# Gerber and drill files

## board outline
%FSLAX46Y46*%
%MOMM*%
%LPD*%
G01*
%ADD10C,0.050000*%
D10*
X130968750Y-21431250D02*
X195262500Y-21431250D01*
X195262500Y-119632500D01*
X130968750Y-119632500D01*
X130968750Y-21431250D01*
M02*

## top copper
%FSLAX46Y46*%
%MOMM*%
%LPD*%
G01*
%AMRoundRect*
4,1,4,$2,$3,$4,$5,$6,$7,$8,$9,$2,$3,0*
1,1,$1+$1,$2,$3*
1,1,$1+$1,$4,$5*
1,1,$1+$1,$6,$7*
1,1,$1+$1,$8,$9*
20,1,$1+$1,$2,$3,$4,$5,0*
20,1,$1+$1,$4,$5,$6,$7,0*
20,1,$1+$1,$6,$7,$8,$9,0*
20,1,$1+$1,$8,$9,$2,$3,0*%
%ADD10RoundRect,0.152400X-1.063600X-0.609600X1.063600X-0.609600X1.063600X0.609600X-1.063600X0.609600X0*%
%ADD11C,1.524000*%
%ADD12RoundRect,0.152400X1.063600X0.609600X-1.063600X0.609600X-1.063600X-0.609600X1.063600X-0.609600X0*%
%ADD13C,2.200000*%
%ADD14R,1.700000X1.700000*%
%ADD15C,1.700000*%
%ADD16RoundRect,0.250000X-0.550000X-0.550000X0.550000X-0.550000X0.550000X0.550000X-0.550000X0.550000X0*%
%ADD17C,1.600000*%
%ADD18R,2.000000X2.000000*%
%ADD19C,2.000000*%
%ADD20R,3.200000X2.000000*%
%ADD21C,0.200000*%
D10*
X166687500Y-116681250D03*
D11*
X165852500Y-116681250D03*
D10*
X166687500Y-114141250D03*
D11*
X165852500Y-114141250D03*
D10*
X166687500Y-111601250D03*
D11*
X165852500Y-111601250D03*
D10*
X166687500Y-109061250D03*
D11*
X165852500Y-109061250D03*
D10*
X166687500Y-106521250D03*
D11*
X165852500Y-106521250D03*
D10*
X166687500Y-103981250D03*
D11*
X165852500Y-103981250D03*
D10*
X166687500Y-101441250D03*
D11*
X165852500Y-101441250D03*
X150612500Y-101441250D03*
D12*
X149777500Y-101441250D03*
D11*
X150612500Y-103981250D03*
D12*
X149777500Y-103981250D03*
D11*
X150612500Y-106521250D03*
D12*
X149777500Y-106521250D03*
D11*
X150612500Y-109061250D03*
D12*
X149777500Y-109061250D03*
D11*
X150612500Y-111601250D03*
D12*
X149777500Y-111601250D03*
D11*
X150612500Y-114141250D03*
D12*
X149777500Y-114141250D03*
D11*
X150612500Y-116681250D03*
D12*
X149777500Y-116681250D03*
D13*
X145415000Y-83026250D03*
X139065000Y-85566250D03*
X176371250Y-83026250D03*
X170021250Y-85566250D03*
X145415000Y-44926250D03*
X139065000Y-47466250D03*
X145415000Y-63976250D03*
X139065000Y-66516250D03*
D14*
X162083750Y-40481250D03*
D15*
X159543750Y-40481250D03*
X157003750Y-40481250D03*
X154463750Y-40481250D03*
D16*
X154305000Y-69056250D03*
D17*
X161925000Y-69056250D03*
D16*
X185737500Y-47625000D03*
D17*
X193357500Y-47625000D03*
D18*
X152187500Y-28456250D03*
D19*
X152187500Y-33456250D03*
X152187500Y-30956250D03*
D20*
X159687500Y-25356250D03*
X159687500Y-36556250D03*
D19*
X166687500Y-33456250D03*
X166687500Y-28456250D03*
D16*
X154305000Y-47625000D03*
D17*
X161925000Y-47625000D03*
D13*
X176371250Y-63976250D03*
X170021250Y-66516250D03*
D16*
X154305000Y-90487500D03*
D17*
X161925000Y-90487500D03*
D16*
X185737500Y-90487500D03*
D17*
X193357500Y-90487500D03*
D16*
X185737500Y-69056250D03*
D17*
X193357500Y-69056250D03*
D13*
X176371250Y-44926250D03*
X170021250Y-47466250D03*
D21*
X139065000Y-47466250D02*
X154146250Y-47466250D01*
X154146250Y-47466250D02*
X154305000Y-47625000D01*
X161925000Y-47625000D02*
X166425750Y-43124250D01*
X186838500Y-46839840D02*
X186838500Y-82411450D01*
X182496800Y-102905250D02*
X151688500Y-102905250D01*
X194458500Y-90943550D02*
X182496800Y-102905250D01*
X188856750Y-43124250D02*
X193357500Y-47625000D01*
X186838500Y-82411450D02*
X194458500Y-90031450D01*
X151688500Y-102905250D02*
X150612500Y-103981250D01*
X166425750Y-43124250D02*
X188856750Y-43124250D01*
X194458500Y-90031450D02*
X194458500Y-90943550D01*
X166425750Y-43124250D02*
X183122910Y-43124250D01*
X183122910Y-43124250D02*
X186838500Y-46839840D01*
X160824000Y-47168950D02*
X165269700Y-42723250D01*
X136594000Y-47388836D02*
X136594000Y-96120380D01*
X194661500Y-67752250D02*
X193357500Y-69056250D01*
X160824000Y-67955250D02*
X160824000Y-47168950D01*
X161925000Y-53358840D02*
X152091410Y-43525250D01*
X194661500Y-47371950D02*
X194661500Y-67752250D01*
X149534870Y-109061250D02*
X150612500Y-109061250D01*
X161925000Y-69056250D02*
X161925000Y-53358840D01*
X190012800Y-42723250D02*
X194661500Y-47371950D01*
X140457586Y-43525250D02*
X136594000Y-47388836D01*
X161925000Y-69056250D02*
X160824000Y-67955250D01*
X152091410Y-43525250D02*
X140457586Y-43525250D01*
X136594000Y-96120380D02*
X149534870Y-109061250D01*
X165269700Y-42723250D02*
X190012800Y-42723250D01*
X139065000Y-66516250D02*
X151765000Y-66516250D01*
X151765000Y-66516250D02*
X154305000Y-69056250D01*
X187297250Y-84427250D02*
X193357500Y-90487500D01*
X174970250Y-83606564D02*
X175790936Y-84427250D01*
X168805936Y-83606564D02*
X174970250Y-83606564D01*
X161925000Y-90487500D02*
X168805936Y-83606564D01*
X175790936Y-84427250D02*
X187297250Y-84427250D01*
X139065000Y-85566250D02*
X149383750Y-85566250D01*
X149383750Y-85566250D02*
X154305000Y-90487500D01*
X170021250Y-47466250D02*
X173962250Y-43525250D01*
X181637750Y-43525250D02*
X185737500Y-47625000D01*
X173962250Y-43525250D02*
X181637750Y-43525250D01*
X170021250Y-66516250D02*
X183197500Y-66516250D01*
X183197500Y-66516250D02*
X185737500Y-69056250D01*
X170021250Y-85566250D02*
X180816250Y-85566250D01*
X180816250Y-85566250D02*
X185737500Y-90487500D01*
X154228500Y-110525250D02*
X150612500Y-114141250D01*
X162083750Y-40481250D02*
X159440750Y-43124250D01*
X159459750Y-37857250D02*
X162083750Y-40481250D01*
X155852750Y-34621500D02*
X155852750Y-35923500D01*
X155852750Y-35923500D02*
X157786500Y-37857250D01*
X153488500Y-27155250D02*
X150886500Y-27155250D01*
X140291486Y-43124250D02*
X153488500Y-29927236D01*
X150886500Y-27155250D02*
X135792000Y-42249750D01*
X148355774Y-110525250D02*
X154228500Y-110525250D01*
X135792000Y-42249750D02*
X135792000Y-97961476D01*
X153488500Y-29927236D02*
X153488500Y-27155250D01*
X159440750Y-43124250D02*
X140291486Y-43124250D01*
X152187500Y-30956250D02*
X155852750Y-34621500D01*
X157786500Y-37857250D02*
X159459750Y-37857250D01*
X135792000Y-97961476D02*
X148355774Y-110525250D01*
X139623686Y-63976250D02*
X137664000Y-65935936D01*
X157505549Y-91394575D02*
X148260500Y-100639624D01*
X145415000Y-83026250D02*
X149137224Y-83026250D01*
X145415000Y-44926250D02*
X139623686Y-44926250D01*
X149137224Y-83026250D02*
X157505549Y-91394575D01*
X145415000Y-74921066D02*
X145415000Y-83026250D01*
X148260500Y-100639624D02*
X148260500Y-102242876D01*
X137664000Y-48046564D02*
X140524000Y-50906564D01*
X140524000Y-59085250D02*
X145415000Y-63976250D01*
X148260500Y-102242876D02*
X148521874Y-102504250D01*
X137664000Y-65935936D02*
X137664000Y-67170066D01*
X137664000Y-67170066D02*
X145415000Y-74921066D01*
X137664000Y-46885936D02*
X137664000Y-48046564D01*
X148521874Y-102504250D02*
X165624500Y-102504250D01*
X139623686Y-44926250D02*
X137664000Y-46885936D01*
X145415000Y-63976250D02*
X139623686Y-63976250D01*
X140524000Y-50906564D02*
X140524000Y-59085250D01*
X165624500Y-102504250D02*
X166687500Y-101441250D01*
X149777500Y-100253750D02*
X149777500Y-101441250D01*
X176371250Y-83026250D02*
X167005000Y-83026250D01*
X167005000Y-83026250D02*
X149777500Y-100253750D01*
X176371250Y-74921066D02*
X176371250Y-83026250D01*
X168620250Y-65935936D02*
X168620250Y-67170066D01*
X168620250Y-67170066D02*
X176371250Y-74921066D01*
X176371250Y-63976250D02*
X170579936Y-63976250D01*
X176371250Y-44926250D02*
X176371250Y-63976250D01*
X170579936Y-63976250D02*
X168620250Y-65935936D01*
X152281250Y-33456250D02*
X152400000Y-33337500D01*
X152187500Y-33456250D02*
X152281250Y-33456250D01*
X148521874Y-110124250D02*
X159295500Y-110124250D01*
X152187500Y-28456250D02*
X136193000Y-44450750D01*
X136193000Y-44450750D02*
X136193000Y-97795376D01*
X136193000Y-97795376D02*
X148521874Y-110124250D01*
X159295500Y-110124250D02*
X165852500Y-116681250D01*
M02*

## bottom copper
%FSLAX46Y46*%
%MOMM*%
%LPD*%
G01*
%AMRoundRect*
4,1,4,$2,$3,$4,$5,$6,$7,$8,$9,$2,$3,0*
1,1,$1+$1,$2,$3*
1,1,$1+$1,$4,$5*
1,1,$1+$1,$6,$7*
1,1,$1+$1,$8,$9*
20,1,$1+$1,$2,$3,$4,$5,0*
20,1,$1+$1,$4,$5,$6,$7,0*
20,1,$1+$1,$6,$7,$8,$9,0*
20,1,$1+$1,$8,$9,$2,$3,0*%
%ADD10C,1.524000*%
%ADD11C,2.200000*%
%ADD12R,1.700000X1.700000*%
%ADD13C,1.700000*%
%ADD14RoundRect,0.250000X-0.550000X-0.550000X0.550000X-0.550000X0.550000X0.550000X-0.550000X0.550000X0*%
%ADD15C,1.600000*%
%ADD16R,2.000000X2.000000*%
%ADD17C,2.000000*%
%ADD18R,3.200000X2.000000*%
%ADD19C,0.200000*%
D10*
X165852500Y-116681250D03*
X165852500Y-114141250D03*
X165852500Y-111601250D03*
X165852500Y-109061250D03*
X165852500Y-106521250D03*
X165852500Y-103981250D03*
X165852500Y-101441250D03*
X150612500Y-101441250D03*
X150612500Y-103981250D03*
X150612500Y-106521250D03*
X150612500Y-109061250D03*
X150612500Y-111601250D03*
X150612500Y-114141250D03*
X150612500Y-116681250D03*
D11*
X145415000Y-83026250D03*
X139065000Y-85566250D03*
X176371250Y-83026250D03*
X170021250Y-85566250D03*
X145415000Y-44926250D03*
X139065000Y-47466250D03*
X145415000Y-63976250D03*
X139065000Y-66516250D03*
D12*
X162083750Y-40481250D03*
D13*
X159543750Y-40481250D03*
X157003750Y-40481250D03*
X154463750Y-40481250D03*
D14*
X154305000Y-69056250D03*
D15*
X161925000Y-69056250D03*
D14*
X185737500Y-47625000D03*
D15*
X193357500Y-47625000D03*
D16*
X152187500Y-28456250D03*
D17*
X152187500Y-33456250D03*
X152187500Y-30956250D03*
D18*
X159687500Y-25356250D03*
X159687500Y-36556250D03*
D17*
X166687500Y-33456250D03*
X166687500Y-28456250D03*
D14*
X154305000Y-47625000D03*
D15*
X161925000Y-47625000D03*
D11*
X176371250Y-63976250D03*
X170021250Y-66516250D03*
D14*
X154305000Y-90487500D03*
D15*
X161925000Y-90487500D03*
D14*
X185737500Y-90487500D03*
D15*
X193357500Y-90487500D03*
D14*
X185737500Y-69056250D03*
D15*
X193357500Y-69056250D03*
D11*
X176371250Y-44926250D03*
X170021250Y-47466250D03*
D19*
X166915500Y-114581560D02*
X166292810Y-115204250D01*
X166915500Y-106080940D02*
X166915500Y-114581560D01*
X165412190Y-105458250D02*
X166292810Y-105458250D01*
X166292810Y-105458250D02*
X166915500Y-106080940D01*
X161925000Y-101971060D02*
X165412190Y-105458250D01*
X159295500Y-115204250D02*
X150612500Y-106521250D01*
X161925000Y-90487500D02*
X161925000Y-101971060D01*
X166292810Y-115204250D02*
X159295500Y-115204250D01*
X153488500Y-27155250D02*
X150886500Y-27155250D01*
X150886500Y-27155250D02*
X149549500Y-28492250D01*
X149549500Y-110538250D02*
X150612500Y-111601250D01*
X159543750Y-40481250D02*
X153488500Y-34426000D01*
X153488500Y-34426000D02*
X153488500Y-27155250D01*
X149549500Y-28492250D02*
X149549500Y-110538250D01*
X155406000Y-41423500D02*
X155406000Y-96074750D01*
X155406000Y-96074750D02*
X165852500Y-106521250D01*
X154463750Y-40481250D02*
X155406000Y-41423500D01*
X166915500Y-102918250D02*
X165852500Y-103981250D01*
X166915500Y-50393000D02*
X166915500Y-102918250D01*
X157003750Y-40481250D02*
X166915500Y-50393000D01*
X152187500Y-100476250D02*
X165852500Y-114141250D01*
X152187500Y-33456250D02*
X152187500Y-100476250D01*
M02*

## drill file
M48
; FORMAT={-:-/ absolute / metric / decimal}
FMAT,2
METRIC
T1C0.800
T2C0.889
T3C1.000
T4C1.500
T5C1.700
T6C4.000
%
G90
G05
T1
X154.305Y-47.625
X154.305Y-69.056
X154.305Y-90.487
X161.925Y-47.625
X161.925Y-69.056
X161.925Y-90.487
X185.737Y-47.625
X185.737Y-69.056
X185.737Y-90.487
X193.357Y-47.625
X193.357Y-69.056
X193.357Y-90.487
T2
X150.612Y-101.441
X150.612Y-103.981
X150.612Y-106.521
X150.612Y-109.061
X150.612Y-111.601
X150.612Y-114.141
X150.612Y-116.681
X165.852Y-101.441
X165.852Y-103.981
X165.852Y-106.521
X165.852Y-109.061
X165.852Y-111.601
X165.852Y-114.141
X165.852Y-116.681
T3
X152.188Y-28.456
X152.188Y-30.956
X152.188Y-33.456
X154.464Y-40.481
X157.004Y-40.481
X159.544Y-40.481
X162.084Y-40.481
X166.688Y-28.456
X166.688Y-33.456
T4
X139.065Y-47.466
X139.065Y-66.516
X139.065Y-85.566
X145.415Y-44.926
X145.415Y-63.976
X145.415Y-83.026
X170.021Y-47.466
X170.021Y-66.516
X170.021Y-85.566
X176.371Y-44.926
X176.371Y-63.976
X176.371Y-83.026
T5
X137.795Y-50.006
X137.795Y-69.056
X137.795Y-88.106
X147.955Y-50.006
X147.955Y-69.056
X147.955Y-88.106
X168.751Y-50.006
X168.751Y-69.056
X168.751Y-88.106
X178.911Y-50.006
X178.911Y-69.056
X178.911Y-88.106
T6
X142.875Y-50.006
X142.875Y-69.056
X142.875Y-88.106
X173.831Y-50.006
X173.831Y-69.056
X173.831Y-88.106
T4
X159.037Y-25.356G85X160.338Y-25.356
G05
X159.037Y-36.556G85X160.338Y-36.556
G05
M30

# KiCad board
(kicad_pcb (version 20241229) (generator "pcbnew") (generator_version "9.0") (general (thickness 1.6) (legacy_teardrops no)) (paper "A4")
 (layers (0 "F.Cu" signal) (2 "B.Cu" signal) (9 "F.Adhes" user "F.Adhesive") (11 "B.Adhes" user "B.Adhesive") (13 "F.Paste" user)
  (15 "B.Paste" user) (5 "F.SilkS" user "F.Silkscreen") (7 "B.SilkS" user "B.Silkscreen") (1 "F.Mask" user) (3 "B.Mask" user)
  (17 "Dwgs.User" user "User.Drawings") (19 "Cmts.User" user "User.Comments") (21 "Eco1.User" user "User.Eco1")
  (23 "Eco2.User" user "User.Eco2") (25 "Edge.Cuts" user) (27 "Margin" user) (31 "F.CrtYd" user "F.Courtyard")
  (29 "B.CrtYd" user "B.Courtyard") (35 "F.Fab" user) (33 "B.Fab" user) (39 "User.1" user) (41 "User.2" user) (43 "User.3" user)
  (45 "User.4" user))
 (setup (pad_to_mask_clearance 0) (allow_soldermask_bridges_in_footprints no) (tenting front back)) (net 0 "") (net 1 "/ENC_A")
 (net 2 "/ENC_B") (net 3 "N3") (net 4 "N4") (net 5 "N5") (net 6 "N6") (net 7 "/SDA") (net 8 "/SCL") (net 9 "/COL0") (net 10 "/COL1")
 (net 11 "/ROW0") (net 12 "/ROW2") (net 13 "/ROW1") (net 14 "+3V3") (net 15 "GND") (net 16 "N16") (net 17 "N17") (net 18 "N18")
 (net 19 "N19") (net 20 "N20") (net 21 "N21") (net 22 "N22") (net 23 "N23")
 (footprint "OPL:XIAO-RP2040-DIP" (layer "F.Cu") (at 158.2325 109.06125 180)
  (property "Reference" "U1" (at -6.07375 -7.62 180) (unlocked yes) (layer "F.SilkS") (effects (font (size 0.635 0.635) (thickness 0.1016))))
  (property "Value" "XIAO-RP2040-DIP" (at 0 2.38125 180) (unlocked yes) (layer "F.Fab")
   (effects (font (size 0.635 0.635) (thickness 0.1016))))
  (pad "1" smd roundrect (at -8.455 -7.62) (size 2.432 1.524) (layers "F.Cu" "F.Mask") (roundrect_rratio 0.1) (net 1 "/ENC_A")
   (thermal_bridge_angle 45))
  (pad "1" thru_hole circle (at -7.62 -7.62) (size 1.524 1.524) (drill 0.889) (layers "*.Cu" "*.Mask") (remove_unused_layers no)
   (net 1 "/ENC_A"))
  (pad "2" smd roundrect (at -8.455 -5.08) (size 2.432 1.524) (layers "F.Cu" "F.Mask") (roundrect_rratio 0.1) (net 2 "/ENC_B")
   (thermal_bridge_angle 45))
  (pad "2" thru_hole circle (at -7.62 -5.08) (size 1.524 1.524) (drill 0.889) (layers "*.Cu" "*.Mask") (remove_unused_layers no)
   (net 2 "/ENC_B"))
  (pad "3" smd roundrect (at -8.455 -2.54) (size 2.432 1.524) (layers "F.Cu" "F.Mask") (roundrect_rratio 0.1) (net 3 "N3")
   (thermal_bridge_angle 45))
  (pad "3" thru_hole circle (at -7.62 -2.54) (size 1.524 1.524) (drill 0.889) (layers "*.Cu" "*.Mask") (remove_unused_layers no)
   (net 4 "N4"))
  (pad "4" smd roundrect (at -8.455 0) (size 2.432 1.524) (layers "F.Cu" "F.Mask") (roundrect_rratio 0.1) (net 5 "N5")
   (thermal_bridge_angle 45))
  (pad "4" thru_hole circle (at -7.62 0) (size 1.524 1.524) (drill 0.889) (layers "*.Cu" "*.Mask") (remove_unused_layers no) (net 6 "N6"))
  (pad "5" smd roundrect (at -8.455 2.54) (size 2.432 1.524) (layers "F.Cu" "F.Mask") (roundrect_rratio 0.1) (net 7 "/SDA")
   (thermal_bridge_angle 45))
  (pad "5" thru_hole circle (at -7.62 2.54) (size 1.524 1.524) (drill 0.889) (layers "*.Cu" "*.Mask") (remove_unused_layers no)
   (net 7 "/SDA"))
  (pad "6" smd roundrect (at -8.455 5.08) (size 2.432 1.524) (layers "F.Cu" "F.Mask") (roundrect_rratio 0.1) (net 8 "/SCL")
   (thermal_bridge_angle 45))
  (pad "6" thru_hole circle (at -7.62 5.08) (size 1.524 1.524) (drill 0.889) (layers "*.Cu" "*.Mask") (remove_unused_layers no)
   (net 8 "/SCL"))
  (pad "7" smd roundrect (at -8.455 7.62) (size 2.432 1.524) (layers "F.Cu" "F.Mask") (roundrect_rratio 0.1) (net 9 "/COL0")
   (thermal_bridge_angle 45))
  (pad "7" thru_hole circle (at -7.62 7.62) (size 1.524 1.524) (drill 0.889) (layers "*.Cu" "*.Mask") (remove_unused_layers no)
   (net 9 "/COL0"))
  (pad "8" thru_hole circle (at 7.62 7.62 180) (size 1.524 1.524) (drill 0.889) (layers "*.Cu" "*.Mask") (remove_unused_layers no)
   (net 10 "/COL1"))
  (pad "8" smd roundrect (at 8.455 7.62 180) (size 2.432 1.524) (layers "F.Cu" "F.Mask") (roundrect_rratio 0.1) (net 10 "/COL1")
   (thermal_bridge_angle 45))
  (pad "9" thru_hole circle (at 7.62 5.08 180) (size 1.524 1.524) (drill 0.889) (layers "*.Cu" "*.Mask") (remove_unused_layers no)
   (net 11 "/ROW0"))
  (pad "9" smd roundrect (at 8.455 5.08 180) (size 2.432 1.524) (layers "F.Cu" "F.Mask") (roundrect_rratio 0.1) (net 11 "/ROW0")
   (thermal_bridge_angle 45))
  (pad "10" thru_hole circle (at 7.62 2.54 180) (size 1.524 1.524) (drill 0.889) (layers "*.Cu" "*.Mask") (remove_unused_layers no)
   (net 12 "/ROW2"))
  (pad "10" smd roundrect (at 8.455 2.54 180) (size 2.432 1.524) (layers "F.Cu" "F.Mask") (roundrect_rratio 0.1) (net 12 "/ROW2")
   (thermal_bridge_angle 45))
  (pad "11" thru_hole circle (at 7.62 0 180) (size 1.524 1.524) (drill 0.889) (layers "*.Cu" "*.Mask") (remove_unused_layers no)
   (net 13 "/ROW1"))
  (pad "11" smd roundrect (at 8.455 0 180) (size 2.432 1.524) (layers "F.Cu" "F.Mask") (roundrect_rratio 0.1) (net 13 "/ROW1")
   (thermal_bridge_angle 45))
  (pad "12" thru_hole circle (at 7.62 -2.54 180) (size 1.524 1.524) (drill 0.889) (layers "*.Cu" "*.Mask") (remove_unused_layers no)
   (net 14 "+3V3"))
  (pad "12" smd roundrect (at 8.455 -2.54 180) (size 2.432 1.524) (layers "F.Cu" "F.Mask") (roundrect_rratio 0.1) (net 14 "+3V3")
   (thermal_bridge_angle 45))
  (pad "13" thru_hole circle (at 7.62 -5.08 180) (size 1.524 1.524) (drill 0.889) (layers "*.Cu" "*.Mask") (remove_unused_layers no)
   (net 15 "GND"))
  (pad "13" smd roundrect (at 8.455 -5.08 180) (size 2.432 1.524) (layers "F.Cu" "F.Mask") (roundrect_rratio 0.1) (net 15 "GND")
   (thermal_bridge_angle 45))
  (pad "14" thru_hole circle (at 7.62 -7.62 180) (size 1.524 1.524) (drill 0.889) (layers "*.Cu" "*.Mask") (remove_unused_layers no)
   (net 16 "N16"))
  (pad "14" smd roundrect (at 8.455 -7.62 180) (size 2.432 1.524) (layers "F.Cu" "F.Mask") (roundrect_rratio 0.1) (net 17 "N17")
   (thermal_bridge_angle 45)))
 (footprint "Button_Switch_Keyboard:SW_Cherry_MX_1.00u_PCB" (layer "F.Cu") (at 145.415 83.02625)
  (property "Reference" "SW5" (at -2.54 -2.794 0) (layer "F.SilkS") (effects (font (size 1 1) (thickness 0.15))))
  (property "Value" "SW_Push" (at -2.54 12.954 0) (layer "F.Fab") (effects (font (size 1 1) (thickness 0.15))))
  (pad "" np_thru_hole circle (at -7.62 5.08) (size 1.7 1.7) (drill 1.7) (layers "*.Cu" "*.Mask"))
  (pad "" np_thru_hole circle (at -2.54 5.08) (size 4 4) (drill 4) (layers "*.Cu" "*.Mask"))
  (pad "" np_thru_hole circle (at 2.54 5.08) (size 1.7 1.7) (drill 1.7) (layers "*.Cu" "*.Mask"))
  (pad "1" thru_hole circle (at 0 0) (size 2.2 2.2) (drill 1.5) (layers "*.Cu" "*.Mask") (remove_unused_layers no) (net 9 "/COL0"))
  (pad "2" thru_hole circle (at -6.35 2.54) (size 2.2 2.2) (drill 1.5) (layers "*.Cu" "*.Mask") (remove_unused_layers no) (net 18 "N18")))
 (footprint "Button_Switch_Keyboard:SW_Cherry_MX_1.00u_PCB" (layer "F.Cu") (at 176.37125 83.02625)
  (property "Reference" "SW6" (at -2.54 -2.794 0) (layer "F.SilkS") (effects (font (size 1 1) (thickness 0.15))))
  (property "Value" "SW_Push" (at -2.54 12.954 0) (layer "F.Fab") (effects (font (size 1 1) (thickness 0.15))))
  (pad "" np_thru_hole circle (at -7.62 5.08) (size 1.7 1.7) (drill 1.7) (layers "*.Cu" "*.Mask"))
  (pad "" np_thru_hole circle (at -2.54 5.08) (size 4 4) (drill 4) (layers "*.Cu" "*.Mask"))
  (pad "" np_thru_hole circle (at 2.54 5.08) (size 1.7 1.7) (drill 1.7) (layers "*.Cu" "*.Mask"))
  (pad "1" thru_hole circle (at 0 0) (size 2.2 2.2) (drill 1.5) (layers "*.Cu" "*.Mask") (remove_unused_layers no) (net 10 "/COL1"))
  (pad "2" thru_hole circle (at -6.35 2.54) (size 2.2 2.2) (drill 1.5) (layers "*.Cu" "*.Mask") (remove_unused_layers no) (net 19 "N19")))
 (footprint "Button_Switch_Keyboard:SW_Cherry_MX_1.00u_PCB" (layer "F.Cu") (at 145.415 44.92625)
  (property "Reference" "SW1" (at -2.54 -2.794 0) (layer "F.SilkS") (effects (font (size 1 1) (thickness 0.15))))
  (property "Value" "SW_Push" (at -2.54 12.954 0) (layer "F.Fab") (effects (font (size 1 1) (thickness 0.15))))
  (pad "" np_thru_hole circle (at -7.62 5.08) (size 1.7 1.7) (drill 1.7) (layers "*.Cu" "*.Mask"))
  (pad "" np_thru_hole circle (at -2.54 5.08) (size 4 4) (drill 4) (layers "*.Cu" "*.Mask"))
  (pad "" np_thru_hole circle (at 2.54 5.08) (size 1.7 1.7) (drill 1.7) (layers "*.Cu" "*.Mask"))
  (pad "1" thru_hole circle (at 0 0) (size 2.2 2.2) (drill 1.5) (layers "*.Cu" "*.Mask") (remove_unused_layers no) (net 9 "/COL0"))
  (pad "2" thru_hole circle (at -6.35 2.54) (size 2.2 2.2) (drill 1.5) (layers "*.Cu" "*.Mask") (remove_unused_layers no) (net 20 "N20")))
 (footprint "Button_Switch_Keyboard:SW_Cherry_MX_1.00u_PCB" (layer "F.Cu") (at 145.415 63.97625)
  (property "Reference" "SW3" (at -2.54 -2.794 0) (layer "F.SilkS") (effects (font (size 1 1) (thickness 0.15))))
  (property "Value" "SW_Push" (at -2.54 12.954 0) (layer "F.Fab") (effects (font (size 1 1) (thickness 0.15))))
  (pad "" np_thru_hole circle (at -7.62 5.08) (size 1.7 1.7) (drill 1.7) (layers "*.Cu" "*.Mask"))
  (pad "" np_thru_hole circle (at -2.54 5.08) (size 4 4) (drill 4) (layers "*.Cu" "*.Mask"))
  (pad "" np_thru_hole circle (at 2.54 5.08) (size 1.7 1.7) (drill 1.7) (layers "*.Cu" "*.Mask"))
  (pad "1" thru_hole circle (at 0 0) (size 2.2 2.2) (drill 1.5) (layers "*.Cu" "*.Mask") (remove_unused_layers no) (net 9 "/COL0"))
  (pad "2" thru_hole circle (at -6.35 2.54) (size 2.2 2.2) (drill 1.5) (layers "*.Cu" "*.Mask") (remove_unused_layers no) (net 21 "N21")))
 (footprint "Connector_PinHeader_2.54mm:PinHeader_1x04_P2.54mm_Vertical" (layer "F.Cu") (at 162.08375 40.48125 -90)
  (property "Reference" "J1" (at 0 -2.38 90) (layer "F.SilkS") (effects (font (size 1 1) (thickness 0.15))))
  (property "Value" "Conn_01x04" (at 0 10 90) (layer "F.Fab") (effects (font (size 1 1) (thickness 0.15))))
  (pad "1" thru_hole rect (at 0 0 270) (size 1.7 1.7) (drill 1) (layers "*.Cu" "*.Mask") (remove_unused_layers no) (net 15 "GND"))
  (pad "2" thru_hole circle (at 0 2.54 270) (size 1.7 1.7) (drill 1) (layers "*.Cu" "*.Mask") (remove_unused_layers no) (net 14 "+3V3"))
  (pad "3" thru_hole circle (at 0 5.08 270) (size 1.7 1.7) (drill 1) (layers "*.Cu" "*.Mask") (remove_unused_layers no) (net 8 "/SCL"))
  (pad "4" thru_hole circle (at 0 7.62 270) (size 1.7 1.7) (drill 1) (layers "*.Cu" "*.Mask") (remove_unused_layers no) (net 7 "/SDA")))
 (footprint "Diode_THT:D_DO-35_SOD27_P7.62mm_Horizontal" (layer "F.Cu") (at 154.305 69.05625)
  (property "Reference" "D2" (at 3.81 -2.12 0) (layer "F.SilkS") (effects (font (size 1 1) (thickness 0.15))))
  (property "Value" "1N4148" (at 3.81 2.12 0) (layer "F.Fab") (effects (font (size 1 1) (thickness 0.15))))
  (pad "1" thru_hole roundrect (at 0 0) (size 1.6 1.6) (drill 0.8) (layers "*.Cu" "*.Mask") (remove_unused_layers no)
   (roundrect_rratio 0.15625) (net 21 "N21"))
  (pad "2" thru_hole circle (at 7.62 0) (size 1.6 1.6) (drill 0.8) (layers "*.Cu" "*.Mask") (remove_unused_layers no) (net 13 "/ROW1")))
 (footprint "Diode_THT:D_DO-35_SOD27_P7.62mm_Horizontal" (layer "F.Cu") (at 185.7375 47.625)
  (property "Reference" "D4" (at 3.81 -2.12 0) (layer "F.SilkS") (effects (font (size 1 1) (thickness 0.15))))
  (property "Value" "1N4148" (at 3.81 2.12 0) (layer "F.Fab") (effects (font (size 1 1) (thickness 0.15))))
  (pad "1" thru_hole roundrect (at 0 0) (size 1.6 1.6) (drill 0.8) (layers "*.Cu" "*.Mask") (remove_unused_layers no)
   (roundrect_rratio 0.15625) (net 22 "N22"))
  (pad "2" thru_hole circle (at 7.62 0) (size 1.6 1.6) (drill 0.8) (layers "*.Cu" "*.Mask") (remove_unused_layers no) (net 11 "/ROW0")))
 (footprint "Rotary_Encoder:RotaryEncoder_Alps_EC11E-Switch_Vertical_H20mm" (layer "F.Cu") (at 152.1875 28.45625)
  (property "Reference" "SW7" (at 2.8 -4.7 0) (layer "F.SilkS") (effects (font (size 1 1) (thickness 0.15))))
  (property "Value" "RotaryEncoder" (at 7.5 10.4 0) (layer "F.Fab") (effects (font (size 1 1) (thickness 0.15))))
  (pad "A" thru_hole rect (at 0 0) (size 2 2) (drill 1) (layers "*.Cu" "*.Mask") (remove_unused_layers no) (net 1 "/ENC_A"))
  (pad "B" thru_hole circle (at 0 5) (size 2 2) (drill 1) (layers "*.Cu" "*.Mask") (remove_unused_layers no) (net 2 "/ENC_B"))
  (pad "C" thru_hole circle (at 0 2.5) (size 2 2) (drill 1) (layers "*.Cu" "*.Mask") (remove_unused_layers no) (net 15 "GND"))
  (pad "MP" thru_hole rect (at 7.5 -3.1) (size 3.2 2) (drill oval 2.8 1.5) (layers "*.Cu" "*.Mask") (remove_unused_layers no))
  (pad "MP" thru_hole rect (at 7.5 8.1) (size 3.2 2) (drill oval 2.8 1.5) (layers "*.Cu" "*.Mask") (remove_unused_layers no))
  (pad "S1" thru_hole circle (at 14.5 5) (size 2 2) (drill 1) (layers "*.Cu" "*.Mask") (remove_unused_layers no))
  (pad "S2" thru_hole circle (at 14.5 0) (size 2 2) (drill 1) (layers "*.Cu" "*.Mask") (remove_unused_layers no)))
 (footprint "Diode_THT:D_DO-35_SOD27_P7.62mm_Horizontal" (layer "F.Cu") (at 154.305 47.625)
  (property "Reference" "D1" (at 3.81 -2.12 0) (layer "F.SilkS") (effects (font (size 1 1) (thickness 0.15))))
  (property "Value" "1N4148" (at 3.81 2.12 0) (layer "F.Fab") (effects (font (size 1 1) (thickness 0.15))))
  (pad "1" thru_hole roundrect (at 0 0) (size 1.6 1.6) (drill 0.8) (layers "*.Cu" "*.Mask") (remove_unused_layers no)
   (roundrect_rratio 0.15625) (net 20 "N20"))
  (pad "2" thru_hole circle (at 7.62 0) (size 1.6 1.6) (drill 0.8) (layers "*.Cu" "*.Mask") (remove_unused_layers no) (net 11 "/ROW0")))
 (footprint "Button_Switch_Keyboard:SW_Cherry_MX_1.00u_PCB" (layer "F.Cu") (at 176.37125 63.97625)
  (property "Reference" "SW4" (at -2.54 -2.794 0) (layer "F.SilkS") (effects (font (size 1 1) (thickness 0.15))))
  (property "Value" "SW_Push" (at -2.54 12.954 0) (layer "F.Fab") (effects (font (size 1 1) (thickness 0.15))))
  (pad "" np_thru_hole circle (at -7.62 5.08) (size 1.7 1.7) (drill 1.7) (layers "*.Cu" "*.Mask"))
  (pad "" np_thru_hole circle (at -2.54 5.08) (size 4 4) (drill 4) (layers "*.Cu" "*.Mask"))
  (pad "" np_thru_hole circle (at 2.54 5.08) (size 1.7 1.7) (drill 1.7) (layers "*.Cu" "*.Mask"))
  (pad "1" thru_hole circle (at 0 0) (size 2.2 2.2) (drill 1.5) (layers "*.Cu" "*.Mask") (remove_unused_layers no) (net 10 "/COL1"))
  (pad "2" thru_hole circle (at -6.35 2.54) (size 2.2 2.2) (drill 1.5) (layers "*.Cu" "*.Mask") (remove_unused_layers no) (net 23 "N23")))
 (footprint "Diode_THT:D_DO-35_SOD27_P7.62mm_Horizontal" (layer "F.Cu") (at 154.305 90.4875)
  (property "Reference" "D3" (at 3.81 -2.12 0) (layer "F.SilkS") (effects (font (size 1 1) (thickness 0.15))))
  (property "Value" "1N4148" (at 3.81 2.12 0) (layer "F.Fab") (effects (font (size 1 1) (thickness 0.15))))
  (pad "1" thru_hole roundrect (at 0 0) (size 1.6 1.6) (drill 0.8) (layers "*.Cu" "*.Mask") (remove_unused_layers no)
   (roundrect_rratio 0.15625) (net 18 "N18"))
  (pad "2" thru_hole circle (at 7.62 0) (size 1.6 1.6) (drill 0.8) (layers "*.Cu" "*.Mask") (remove_unused_layers no) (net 12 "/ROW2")))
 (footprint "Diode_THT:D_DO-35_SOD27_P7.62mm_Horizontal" (layer "F.Cu") (at 185.7375 90.4875)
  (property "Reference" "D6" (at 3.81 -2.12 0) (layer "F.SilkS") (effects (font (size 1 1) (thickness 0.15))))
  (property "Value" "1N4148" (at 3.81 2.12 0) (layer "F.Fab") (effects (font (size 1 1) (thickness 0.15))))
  (pad "1" thru_hole roundrect (at 0 0) (size 1.6 1.6) (drill 0.8) (layers "*.Cu" "*.Mask") (remove_unused_layers no)
   (roundrect_rratio 0.15625) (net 19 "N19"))
  (pad "2" thru_hole circle (at 7.62 0) (size 1.6 1.6) (drill 0.8) (layers "*.Cu" "*.Mask") (remove_unused_layers no) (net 12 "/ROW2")))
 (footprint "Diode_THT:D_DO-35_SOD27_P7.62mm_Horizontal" (layer "F.Cu") (at 185.7375 69.05625)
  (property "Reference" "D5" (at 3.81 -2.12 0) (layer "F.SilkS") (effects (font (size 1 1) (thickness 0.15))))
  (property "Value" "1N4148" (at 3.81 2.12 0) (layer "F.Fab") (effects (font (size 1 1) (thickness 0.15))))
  (pad "1" thru_hole roundrect (at 0 0) (size 1.6 1.6) (drill 0.8) (layers "*.Cu" "*.Mask") (remove_unused_layers no)
   (roundrect_rratio 0.15625) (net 23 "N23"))
  (pad "2" thru_hole circle (at 7.62 0) (size 1.6 1.6) (drill 0.8) (layers "*.Cu" "*.Mask") (remove_unused_layers no) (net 13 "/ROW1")))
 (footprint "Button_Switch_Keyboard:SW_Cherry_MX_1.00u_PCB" (layer "F.Cu") (at 176.37125 44.92625)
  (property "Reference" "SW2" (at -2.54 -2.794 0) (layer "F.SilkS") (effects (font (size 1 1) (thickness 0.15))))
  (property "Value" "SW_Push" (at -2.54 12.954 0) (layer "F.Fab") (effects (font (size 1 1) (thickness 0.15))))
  (pad "" np_thru_hole circle (at -7.62 5.08) (size 1.7 1.7) (drill 1.7) (layers "*.Cu" "*.Mask"))
  (pad "" np_thru_hole circle (at -2.54 5.08) (size 4 4) (drill 4) (layers "*.Cu" "*.Mask"))
  (pad "" np_thru_hole circle (at 2.54 5.08) (size 1.7 1.7) (drill 1.7) (layers "*.Cu" "*.Mask"))
  (pad "1" thru_hole circle (at 0 0) (size 2.2 2.2) (drill 1.5) (layers "*.Cu" "*.Mask") (remove_unused_layers no) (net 10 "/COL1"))
  (pad "2" thru_hole circle (at -6.35 2.54) (size 2.2 2.2) (drill 1.5) (layers "*.Cu" "*.Mask") (remove_unused_layers no) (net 22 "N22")))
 (gr_rect (start 130.96875 21.43125) (end 195.2625 119.6325) (stroke (width 0.05) (type default)) (fill no) (layer "Edge.Cuts"))
 (segment (start 139.065 47.46625) (end 154.14625 47.46625) (width 0.2) (layer "F.Cu") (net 20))
 (segment (start 154.14625 47.46625) (end 154.305 47.625) (width 0.2) (layer "F.Cu") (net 20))
 (segment (start 161.925 47.625) (end 166.42575 43.12425) (width 0.2) (layer "F.Cu") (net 11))
 (segment (start 186.8385 46.83984) (end 186.8385 82.41145) (width 0.2) (layer "F.Cu") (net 11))
 (segment (start 182.4968 102.90525) (end 151.6885 102.90525) (width 0.2) (layer "F.Cu") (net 11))
 (segment (start 194.4585 90.94355) (end 182.4968 102.90525) (width 0.2) (layer "F.Cu") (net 11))
 (segment (start 188.85675 43.12425) (end 193.3575 47.625) (width 0.2) (layer "F.Cu") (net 11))
 (segment (start 186.8385 82.41145) (end 194.4585 90.03145) (width 0.2) (layer "F.Cu") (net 11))
 (segment (start 151.6885 102.90525) (end 150.6125 103.98125) (width 0.2) (layer "F.Cu") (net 11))
 (segment (start 166.42575 43.12425) (end 188.85675 43.12425) (width 0.2) (layer "F.Cu") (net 11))
 (segment (start 194.4585 90.03145) (end 194.4585 90.94355) (width 0.2) (layer "F.Cu") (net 11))
 (segment (start 166.42575 43.12425) (end 183.12291 43.12425) (width 0.2) (layer "F.Cu") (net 11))
 (segment (start 183.12291 43.12425) (end 186.8385 46.83984) (width 0.2) (layer "F.Cu") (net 11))
 (segment (start 160.824 47.16895) (end 165.2697 42.72325) (width 0.2) (layer "F.Cu") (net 13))
 (segment (start 136.594 47.388836) (end 136.594 96.12038) (width 0.2) (layer "F.Cu") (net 13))
 (segment (start 194.6615 67.75225) (end 193.3575 69.05625) (width 0.2) (layer "F.Cu") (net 13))
 (segment (start 160.824 67.95525) (end 160.824 47.16895) (width 0.2) (layer "F.Cu") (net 13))
 (segment (start 161.925 53.35884) (end 152.09141 43.52525) (width 0.2) (layer "F.Cu") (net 13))
 (segment (start 194.6615 47.37195) (end 194.6615 67.75225) (width 0.2) (layer "F.Cu") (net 13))
 (segment (start 149.53487 109.06125) (end 150.6125 109.06125) (width 0.2) (layer "F.Cu") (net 13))
 (segment (start 161.925 69.05625) (end 161.925 53.35884) (width 0.2) (layer "F.Cu") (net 13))
 (segment (start 190.0128 42.72325) (end 194.6615 47.37195) (width 0.2) (layer "F.Cu") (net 13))
 (segment (start 140.457586 43.52525) (end 136.594 47.388836) (width 0.2) (layer "F.Cu") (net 13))
 (segment (start 161.925 69.05625) (end 160.824 67.95525) (width 0.2) (layer "F.Cu") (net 13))
 (segment (start 152.09141 43.52525) (end 140.457586 43.52525) (width 0.2) (layer "F.Cu") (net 13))
 (segment (start 136.594 96.12038) (end 149.53487 109.06125) (width 0.2) (layer "F.Cu") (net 13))
 (segment (start 165.2697 42.72325) (end 190.0128 42.72325) (width 0.2) (layer "F.Cu") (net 13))
 (segment (start 139.065 66.51625) (end 151.765 66.51625) (width 0.2) (layer "F.Cu") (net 21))
 (segment (start 151.765 66.51625) (end 154.305 69.05625) (width 0.2) (layer "F.Cu") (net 21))
 (segment (start 187.29725 84.42725) (end 193.3575 90.4875) (width 0.2) (layer "F.Cu") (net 12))
 (segment (start 174.97025 83.606564) (end 175.790936 84.42725) (width 0.2) (layer "F.Cu") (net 12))
 (segment (start 168.805936 83.606564) (end 174.97025 83.606564) (width 0.2) (layer "F.Cu") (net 12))
 (segment (start 161.925 90.4875) (end 168.805936 83.606564) (width 0.2) (layer "F.Cu") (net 12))
 (segment (start 175.790936 84.42725) (end 187.29725 84.42725) (width 0.2) (layer "F.Cu") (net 12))
 (segment (start 166.9155 114.58156) (end 166.29281 115.20425) (width 0.2) (layer "B.Cu") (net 12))
 (segment (start 166.9155 106.08094) (end 166.9155 114.58156) (width 0.2) (layer "B.Cu") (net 12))
 (segment (start 165.41219 105.45825) (end 166.29281 105.45825) (width 0.2) (layer "B.Cu") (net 12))
 (segment (start 166.29281 105.45825) (end 166.9155 106.08094) (width 0.2) (layer "B.Cu") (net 12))
 (segment (start 161.925 101.97106) (end 165.41219 105.45825) (width 0.2) (layer "B.Cu") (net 12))
 (segment (start 159.2955 115.20425) (end 150.6125 106.52125) (width 0.2) (layer "B.Cu") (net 12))
 (segment (start 161.925 90.4875) (end 161.925 101.97106) (width 0.2) (layer "B.Cu") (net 12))
 (segment (start 166.29281 115.20425) (end 159.2955 115.20425) (width 0.2) (layer "B.Cu") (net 12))
 (segment (start 139.065 85.56625) (end 149.38375 85.56625) (width 0.2) (layer "F.Cu") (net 18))
 (segment (start 149.38375 85.56625) (end 154.305 90.4875) (width 0.2) (layer "F.Cu") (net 18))
 (segment (start 170.02125 47.46625) (end 173.96225 43.52525) (width 0.2) (layer "F.Cu") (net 22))
 (segment (start 181.63775 43.52525) (end 185.7375 47.625) (width 0.2) (layer "F.Cu") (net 22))
 (segment (start 173.96225 43.52525) (end 181.63775 43.52525) (width 0.2) (layer "F.Cu") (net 22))
 (segment (start 170.02125 66.51625) (end 183.1975 66.51625) (width 0.2) (layer "F.Cu") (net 23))
 (segment (start 183.1975 66.51625) (end 185.7375 69.05625) (width 0.2) (layer "F.Cu") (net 23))
 (segment (start 170.02125 85.56625) (end 180.81625 85.56625) (width 0.2) (layer "F.Cu") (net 19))
 (segment (start 180.81625 85.56625) (end 185.7375 90.4875) (width 0.2) (layer "F.Cu") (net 19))
 (segment (start 154.2285 110.52525) (end 150.6125 114.14125) (width 0.2) (layer "F.Cu") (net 15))
 (segment (start 162.08375 40.48125) (end 159.44075 43.12425) (width 0.2) (layer "F.Cu") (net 15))
 (segment (start 159.45975 37.85725) (end 162.08375 40.48125) (width 0.2) (layer "F.Cu") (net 15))
 (segment (start 155.85275 34.6215) (end 155.85275 35.9235) (width 0.2) (layer "F.Cu") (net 15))
 (segment (start 155.85275 35.9235) (end 157.7865 37.85725) (width 0.2) (layer "F.Cu") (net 15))
 (segment (start 153.4885 27.15525) (end 150.8865 27.15525) (width 0.2) (layer "F.Cu") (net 15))
 (segment (start 140.291486 43.12425) (end 153.4885 29.927236) (width 0.2) (layer "F.Cu") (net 15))
 (segment (start 150.8865 27.15525) (end 135.792 42.24975) (width 0.2) (layer "F.Cu") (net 15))
 (segment (start 148.355774 110.52525) (end 154.2285 110.52525) (width 0.2) (layer "F.Cu") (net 15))
 (segment (start 135.792 42.24975) (end 135.792 97.961476) (width 0.2) (layer "F.Cu") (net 15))
 (segment (start 153.4885 29.927236) (end 153.4885 27.15525) (width 0.2) (layer "F.Cu") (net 15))
 (segment (start 159.44075 43.12425) (end 140.291486 43.12425) (width 0.2) (layer "F.Cu") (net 15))
 (segment (start 152.1875 30.95625) (end 155.85275 34.6215) (width 0.2) (layer "F.Cu") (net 15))
 (segment (start 157.7865 37.85725) (end 159.45975 37.85725) (width 0.2) (layer "F.Cu") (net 15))
 (segment (start 135.792 97.961476) (end 148.355774 110.52525) (width 0.2) (layer "F.Cu") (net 15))
 (segment (start 153.4885 27.15525) (end 150.8865 27.15525) (width 0.2) (layer "B.Cu") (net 14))
 (segment (start 150.8865 27.15525) (end 149.5495 28.49225) (width 0.2) (layer "B.Cu") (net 14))
 (segment (start 149.5495 110.53825) (end 150.6125 111.60125) (width 0.2) (layer "B.Cu") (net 14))
 (segment (start 159.54375 40.48125) (end 153.4885 34.426) (width 0.2) (layer "B.Cu") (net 14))
 (segment (start 153.4885 34.426) (end 153.4885 27.15525) (width 0.2) (layer "B.Cu") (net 14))
 (segment (start 149.5495 28.49225) (end 149.5495 110.53825) (width 0.2) (layer "B.Cu") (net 14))
 (segment (start 155.406 41.4235) (end 155.406 96.07475) (width 0.2) (layer "B.Cu") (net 7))
 (segment (start 155.406 96.07475) (end 165.8525 106.52125) (width 0.2) (layer "B.Cu") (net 7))
 (segment (start 154.46375 40.48125) (end 155.406 41.4235) (width 0.2) (layer "B.Cu") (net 7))
 (segment (start 166.9155 102.91825) (end 165.8525 103.98125) (width 0.2) (layer "B.Cu") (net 8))
 (segment (start 166.9155 50.393) (end 166.9155 102.91825) (width 0.2) (layer "B.Cu") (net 8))
 (segment (start 157.00375 40.48125) (end 166.9155 50.393) (width 0.2) (layer "B.Cu") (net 8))
 (segment (start 139.623686 63.97625) (end 137.664 65.935936) (width 0.2) (layer "F.Cu") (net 9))
 (segment (start 157.505549 91.394575) (end 148.2605 100.639624) (width 0.2) (layer "F.Cu") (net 9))
 (segment (start 145.415 83.02625) (end 149.137224 83.02625) (width 0.2) (layer "F.Cu") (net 9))
 (segment (start 145.415 44.92625) (end 139.623686 44.92625) (width 0.2) (layer "F.Cu") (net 9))
 (segment (start 149.137224 83.02625) (end 157.505549 91.394575) (width 0.2) (layer "F.Cu") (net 9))
 (segment (start 145.415 74.921066) (end 145.415 83.02625) (width 0.2) (layer "F.Cu") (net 9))
 (segment (start 148.2605 100.639624) (end 148.2605 102.242876) (width 0.2) (layer "F.Cu") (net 9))
 (segment (start 137.664 48.046564) (end 140.524 50.906564) (width 0.2) (layer "F.Cu") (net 9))
 (segment (start 140.524 59.08525) (end 145.415 63.97625) (width 0.2) (layer "F.Cu") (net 9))
 (segment (start 148.2605 102.242876) (end 148.521874 102.50425) (width 0.2) (layer "F.Cu") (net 9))
 (segment (start 137.664 65.935936) (end 137.664 67.170066) (width 0.2) (layer "F.Cu") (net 9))
 (segment (start 137.664 67.170066) (end 145.415 74.921066) (width 0.2) (layer "F.Cu") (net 9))
 (segment (start 137.664 46.885936) (end 137.664 48.046564) (width 0.2) (layer "F.Cu") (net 9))
 (segment (start 148.521874 102.50425) (end 165.6245 102.50425) (width 0.2) (layer "F.Cu") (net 9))
 (segment (start 139.623686 44.92625) (end 137.664 46.885936) (width 0.2) (layer "F.Cu") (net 9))
 (segment (start 145.415 63.97625) (end 139.623686 63.97625) (width 0.2) (layer "F.Cu") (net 9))
 (segment (start 140.524 50.906564) (end 140.524 59.08525) (width 0.2) (layer "F.Cu") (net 9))
 (segment (start 165.6245 102.50425) (end 166.6875 101.44125) (width 0.2) (layer "F.Cu") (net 9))
 (segment (start 149.7775 100.25375) (end 149.7775 101.44125) (width 0.2) (layer "F.Cu") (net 10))
 (segment (start 176.37125 83.02625) (end 167.005 83.02625) (width 0.2) (layer "F.Cu") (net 10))
 (segment (start 167.005 83.02625) (end 149.7775 100.25375) (width 0.2) (layer "F.Cu") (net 10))
 (segment (start 176.37125 74.921066) (end 176.37125 83.02625) (width 0.2) (layer "F.Cu") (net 10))
 (segment (start 168.62025 65.935936) (end 168.62025 67.170066) (width 0.2) (layer "F.Cu") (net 10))
 (segment (start 168.62025 67.170066) (end 176.37125 74.921066) (width 0.2) (layer "F.Cu") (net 10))
 (segment (start 176.37125 63.97625) (end 170.579936 63.97625) (width 0.2) (layer "F.Cu") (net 10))
 (segment (start 176.37125 44.92625) (end 176.37125 63.97625) (width 0.2) (layer "F.Cu") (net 10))
 (segment (start 170.579936 63.97625) (end 168.62025 65.935936) (width 0.2) (layer "F.Cu") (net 10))
 (segment (start 152.28125 33.45625) (end 152.4 33.3375) (width 0.2) (layer "F.Cu") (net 2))
 (segment (start 152.1875 33.45625) (end 152.28125 33.45625) (width 0.2) (layer "F.Cu") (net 2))
 (segment (start 152.1875 100.47625) (end 165.8525 114.14125) (width 0.2) (layer "B.Cu") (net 2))
 (segment (start 152.1875 33.45625) (end 152.1875 100.47625) (width 0.2) (layer "B.Cu") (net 2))
 (segment (start 148.521874 110.12425) (end 159.2955 110.12425) (width 0.2) (layer "F.Cu") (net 1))
 (segment (start 152.1875 28.45625) (end 136.193 44.45075) (width 0.2) (layer "F.Cu") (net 1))
 (segment (start 136.193 44.45075) (end 136.193 97.795376) (width 0.2) (layer "F.Cu") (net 1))
 (segment (start 136.193 97.795376) (end 148.521874 110.12425) (width 0.2) (layer "F.Cu") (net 1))
 (segment (start 159.2955 110.12425) (end 165.8525 116.68125) (width 0.2) (layer "F.Cu") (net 1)))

